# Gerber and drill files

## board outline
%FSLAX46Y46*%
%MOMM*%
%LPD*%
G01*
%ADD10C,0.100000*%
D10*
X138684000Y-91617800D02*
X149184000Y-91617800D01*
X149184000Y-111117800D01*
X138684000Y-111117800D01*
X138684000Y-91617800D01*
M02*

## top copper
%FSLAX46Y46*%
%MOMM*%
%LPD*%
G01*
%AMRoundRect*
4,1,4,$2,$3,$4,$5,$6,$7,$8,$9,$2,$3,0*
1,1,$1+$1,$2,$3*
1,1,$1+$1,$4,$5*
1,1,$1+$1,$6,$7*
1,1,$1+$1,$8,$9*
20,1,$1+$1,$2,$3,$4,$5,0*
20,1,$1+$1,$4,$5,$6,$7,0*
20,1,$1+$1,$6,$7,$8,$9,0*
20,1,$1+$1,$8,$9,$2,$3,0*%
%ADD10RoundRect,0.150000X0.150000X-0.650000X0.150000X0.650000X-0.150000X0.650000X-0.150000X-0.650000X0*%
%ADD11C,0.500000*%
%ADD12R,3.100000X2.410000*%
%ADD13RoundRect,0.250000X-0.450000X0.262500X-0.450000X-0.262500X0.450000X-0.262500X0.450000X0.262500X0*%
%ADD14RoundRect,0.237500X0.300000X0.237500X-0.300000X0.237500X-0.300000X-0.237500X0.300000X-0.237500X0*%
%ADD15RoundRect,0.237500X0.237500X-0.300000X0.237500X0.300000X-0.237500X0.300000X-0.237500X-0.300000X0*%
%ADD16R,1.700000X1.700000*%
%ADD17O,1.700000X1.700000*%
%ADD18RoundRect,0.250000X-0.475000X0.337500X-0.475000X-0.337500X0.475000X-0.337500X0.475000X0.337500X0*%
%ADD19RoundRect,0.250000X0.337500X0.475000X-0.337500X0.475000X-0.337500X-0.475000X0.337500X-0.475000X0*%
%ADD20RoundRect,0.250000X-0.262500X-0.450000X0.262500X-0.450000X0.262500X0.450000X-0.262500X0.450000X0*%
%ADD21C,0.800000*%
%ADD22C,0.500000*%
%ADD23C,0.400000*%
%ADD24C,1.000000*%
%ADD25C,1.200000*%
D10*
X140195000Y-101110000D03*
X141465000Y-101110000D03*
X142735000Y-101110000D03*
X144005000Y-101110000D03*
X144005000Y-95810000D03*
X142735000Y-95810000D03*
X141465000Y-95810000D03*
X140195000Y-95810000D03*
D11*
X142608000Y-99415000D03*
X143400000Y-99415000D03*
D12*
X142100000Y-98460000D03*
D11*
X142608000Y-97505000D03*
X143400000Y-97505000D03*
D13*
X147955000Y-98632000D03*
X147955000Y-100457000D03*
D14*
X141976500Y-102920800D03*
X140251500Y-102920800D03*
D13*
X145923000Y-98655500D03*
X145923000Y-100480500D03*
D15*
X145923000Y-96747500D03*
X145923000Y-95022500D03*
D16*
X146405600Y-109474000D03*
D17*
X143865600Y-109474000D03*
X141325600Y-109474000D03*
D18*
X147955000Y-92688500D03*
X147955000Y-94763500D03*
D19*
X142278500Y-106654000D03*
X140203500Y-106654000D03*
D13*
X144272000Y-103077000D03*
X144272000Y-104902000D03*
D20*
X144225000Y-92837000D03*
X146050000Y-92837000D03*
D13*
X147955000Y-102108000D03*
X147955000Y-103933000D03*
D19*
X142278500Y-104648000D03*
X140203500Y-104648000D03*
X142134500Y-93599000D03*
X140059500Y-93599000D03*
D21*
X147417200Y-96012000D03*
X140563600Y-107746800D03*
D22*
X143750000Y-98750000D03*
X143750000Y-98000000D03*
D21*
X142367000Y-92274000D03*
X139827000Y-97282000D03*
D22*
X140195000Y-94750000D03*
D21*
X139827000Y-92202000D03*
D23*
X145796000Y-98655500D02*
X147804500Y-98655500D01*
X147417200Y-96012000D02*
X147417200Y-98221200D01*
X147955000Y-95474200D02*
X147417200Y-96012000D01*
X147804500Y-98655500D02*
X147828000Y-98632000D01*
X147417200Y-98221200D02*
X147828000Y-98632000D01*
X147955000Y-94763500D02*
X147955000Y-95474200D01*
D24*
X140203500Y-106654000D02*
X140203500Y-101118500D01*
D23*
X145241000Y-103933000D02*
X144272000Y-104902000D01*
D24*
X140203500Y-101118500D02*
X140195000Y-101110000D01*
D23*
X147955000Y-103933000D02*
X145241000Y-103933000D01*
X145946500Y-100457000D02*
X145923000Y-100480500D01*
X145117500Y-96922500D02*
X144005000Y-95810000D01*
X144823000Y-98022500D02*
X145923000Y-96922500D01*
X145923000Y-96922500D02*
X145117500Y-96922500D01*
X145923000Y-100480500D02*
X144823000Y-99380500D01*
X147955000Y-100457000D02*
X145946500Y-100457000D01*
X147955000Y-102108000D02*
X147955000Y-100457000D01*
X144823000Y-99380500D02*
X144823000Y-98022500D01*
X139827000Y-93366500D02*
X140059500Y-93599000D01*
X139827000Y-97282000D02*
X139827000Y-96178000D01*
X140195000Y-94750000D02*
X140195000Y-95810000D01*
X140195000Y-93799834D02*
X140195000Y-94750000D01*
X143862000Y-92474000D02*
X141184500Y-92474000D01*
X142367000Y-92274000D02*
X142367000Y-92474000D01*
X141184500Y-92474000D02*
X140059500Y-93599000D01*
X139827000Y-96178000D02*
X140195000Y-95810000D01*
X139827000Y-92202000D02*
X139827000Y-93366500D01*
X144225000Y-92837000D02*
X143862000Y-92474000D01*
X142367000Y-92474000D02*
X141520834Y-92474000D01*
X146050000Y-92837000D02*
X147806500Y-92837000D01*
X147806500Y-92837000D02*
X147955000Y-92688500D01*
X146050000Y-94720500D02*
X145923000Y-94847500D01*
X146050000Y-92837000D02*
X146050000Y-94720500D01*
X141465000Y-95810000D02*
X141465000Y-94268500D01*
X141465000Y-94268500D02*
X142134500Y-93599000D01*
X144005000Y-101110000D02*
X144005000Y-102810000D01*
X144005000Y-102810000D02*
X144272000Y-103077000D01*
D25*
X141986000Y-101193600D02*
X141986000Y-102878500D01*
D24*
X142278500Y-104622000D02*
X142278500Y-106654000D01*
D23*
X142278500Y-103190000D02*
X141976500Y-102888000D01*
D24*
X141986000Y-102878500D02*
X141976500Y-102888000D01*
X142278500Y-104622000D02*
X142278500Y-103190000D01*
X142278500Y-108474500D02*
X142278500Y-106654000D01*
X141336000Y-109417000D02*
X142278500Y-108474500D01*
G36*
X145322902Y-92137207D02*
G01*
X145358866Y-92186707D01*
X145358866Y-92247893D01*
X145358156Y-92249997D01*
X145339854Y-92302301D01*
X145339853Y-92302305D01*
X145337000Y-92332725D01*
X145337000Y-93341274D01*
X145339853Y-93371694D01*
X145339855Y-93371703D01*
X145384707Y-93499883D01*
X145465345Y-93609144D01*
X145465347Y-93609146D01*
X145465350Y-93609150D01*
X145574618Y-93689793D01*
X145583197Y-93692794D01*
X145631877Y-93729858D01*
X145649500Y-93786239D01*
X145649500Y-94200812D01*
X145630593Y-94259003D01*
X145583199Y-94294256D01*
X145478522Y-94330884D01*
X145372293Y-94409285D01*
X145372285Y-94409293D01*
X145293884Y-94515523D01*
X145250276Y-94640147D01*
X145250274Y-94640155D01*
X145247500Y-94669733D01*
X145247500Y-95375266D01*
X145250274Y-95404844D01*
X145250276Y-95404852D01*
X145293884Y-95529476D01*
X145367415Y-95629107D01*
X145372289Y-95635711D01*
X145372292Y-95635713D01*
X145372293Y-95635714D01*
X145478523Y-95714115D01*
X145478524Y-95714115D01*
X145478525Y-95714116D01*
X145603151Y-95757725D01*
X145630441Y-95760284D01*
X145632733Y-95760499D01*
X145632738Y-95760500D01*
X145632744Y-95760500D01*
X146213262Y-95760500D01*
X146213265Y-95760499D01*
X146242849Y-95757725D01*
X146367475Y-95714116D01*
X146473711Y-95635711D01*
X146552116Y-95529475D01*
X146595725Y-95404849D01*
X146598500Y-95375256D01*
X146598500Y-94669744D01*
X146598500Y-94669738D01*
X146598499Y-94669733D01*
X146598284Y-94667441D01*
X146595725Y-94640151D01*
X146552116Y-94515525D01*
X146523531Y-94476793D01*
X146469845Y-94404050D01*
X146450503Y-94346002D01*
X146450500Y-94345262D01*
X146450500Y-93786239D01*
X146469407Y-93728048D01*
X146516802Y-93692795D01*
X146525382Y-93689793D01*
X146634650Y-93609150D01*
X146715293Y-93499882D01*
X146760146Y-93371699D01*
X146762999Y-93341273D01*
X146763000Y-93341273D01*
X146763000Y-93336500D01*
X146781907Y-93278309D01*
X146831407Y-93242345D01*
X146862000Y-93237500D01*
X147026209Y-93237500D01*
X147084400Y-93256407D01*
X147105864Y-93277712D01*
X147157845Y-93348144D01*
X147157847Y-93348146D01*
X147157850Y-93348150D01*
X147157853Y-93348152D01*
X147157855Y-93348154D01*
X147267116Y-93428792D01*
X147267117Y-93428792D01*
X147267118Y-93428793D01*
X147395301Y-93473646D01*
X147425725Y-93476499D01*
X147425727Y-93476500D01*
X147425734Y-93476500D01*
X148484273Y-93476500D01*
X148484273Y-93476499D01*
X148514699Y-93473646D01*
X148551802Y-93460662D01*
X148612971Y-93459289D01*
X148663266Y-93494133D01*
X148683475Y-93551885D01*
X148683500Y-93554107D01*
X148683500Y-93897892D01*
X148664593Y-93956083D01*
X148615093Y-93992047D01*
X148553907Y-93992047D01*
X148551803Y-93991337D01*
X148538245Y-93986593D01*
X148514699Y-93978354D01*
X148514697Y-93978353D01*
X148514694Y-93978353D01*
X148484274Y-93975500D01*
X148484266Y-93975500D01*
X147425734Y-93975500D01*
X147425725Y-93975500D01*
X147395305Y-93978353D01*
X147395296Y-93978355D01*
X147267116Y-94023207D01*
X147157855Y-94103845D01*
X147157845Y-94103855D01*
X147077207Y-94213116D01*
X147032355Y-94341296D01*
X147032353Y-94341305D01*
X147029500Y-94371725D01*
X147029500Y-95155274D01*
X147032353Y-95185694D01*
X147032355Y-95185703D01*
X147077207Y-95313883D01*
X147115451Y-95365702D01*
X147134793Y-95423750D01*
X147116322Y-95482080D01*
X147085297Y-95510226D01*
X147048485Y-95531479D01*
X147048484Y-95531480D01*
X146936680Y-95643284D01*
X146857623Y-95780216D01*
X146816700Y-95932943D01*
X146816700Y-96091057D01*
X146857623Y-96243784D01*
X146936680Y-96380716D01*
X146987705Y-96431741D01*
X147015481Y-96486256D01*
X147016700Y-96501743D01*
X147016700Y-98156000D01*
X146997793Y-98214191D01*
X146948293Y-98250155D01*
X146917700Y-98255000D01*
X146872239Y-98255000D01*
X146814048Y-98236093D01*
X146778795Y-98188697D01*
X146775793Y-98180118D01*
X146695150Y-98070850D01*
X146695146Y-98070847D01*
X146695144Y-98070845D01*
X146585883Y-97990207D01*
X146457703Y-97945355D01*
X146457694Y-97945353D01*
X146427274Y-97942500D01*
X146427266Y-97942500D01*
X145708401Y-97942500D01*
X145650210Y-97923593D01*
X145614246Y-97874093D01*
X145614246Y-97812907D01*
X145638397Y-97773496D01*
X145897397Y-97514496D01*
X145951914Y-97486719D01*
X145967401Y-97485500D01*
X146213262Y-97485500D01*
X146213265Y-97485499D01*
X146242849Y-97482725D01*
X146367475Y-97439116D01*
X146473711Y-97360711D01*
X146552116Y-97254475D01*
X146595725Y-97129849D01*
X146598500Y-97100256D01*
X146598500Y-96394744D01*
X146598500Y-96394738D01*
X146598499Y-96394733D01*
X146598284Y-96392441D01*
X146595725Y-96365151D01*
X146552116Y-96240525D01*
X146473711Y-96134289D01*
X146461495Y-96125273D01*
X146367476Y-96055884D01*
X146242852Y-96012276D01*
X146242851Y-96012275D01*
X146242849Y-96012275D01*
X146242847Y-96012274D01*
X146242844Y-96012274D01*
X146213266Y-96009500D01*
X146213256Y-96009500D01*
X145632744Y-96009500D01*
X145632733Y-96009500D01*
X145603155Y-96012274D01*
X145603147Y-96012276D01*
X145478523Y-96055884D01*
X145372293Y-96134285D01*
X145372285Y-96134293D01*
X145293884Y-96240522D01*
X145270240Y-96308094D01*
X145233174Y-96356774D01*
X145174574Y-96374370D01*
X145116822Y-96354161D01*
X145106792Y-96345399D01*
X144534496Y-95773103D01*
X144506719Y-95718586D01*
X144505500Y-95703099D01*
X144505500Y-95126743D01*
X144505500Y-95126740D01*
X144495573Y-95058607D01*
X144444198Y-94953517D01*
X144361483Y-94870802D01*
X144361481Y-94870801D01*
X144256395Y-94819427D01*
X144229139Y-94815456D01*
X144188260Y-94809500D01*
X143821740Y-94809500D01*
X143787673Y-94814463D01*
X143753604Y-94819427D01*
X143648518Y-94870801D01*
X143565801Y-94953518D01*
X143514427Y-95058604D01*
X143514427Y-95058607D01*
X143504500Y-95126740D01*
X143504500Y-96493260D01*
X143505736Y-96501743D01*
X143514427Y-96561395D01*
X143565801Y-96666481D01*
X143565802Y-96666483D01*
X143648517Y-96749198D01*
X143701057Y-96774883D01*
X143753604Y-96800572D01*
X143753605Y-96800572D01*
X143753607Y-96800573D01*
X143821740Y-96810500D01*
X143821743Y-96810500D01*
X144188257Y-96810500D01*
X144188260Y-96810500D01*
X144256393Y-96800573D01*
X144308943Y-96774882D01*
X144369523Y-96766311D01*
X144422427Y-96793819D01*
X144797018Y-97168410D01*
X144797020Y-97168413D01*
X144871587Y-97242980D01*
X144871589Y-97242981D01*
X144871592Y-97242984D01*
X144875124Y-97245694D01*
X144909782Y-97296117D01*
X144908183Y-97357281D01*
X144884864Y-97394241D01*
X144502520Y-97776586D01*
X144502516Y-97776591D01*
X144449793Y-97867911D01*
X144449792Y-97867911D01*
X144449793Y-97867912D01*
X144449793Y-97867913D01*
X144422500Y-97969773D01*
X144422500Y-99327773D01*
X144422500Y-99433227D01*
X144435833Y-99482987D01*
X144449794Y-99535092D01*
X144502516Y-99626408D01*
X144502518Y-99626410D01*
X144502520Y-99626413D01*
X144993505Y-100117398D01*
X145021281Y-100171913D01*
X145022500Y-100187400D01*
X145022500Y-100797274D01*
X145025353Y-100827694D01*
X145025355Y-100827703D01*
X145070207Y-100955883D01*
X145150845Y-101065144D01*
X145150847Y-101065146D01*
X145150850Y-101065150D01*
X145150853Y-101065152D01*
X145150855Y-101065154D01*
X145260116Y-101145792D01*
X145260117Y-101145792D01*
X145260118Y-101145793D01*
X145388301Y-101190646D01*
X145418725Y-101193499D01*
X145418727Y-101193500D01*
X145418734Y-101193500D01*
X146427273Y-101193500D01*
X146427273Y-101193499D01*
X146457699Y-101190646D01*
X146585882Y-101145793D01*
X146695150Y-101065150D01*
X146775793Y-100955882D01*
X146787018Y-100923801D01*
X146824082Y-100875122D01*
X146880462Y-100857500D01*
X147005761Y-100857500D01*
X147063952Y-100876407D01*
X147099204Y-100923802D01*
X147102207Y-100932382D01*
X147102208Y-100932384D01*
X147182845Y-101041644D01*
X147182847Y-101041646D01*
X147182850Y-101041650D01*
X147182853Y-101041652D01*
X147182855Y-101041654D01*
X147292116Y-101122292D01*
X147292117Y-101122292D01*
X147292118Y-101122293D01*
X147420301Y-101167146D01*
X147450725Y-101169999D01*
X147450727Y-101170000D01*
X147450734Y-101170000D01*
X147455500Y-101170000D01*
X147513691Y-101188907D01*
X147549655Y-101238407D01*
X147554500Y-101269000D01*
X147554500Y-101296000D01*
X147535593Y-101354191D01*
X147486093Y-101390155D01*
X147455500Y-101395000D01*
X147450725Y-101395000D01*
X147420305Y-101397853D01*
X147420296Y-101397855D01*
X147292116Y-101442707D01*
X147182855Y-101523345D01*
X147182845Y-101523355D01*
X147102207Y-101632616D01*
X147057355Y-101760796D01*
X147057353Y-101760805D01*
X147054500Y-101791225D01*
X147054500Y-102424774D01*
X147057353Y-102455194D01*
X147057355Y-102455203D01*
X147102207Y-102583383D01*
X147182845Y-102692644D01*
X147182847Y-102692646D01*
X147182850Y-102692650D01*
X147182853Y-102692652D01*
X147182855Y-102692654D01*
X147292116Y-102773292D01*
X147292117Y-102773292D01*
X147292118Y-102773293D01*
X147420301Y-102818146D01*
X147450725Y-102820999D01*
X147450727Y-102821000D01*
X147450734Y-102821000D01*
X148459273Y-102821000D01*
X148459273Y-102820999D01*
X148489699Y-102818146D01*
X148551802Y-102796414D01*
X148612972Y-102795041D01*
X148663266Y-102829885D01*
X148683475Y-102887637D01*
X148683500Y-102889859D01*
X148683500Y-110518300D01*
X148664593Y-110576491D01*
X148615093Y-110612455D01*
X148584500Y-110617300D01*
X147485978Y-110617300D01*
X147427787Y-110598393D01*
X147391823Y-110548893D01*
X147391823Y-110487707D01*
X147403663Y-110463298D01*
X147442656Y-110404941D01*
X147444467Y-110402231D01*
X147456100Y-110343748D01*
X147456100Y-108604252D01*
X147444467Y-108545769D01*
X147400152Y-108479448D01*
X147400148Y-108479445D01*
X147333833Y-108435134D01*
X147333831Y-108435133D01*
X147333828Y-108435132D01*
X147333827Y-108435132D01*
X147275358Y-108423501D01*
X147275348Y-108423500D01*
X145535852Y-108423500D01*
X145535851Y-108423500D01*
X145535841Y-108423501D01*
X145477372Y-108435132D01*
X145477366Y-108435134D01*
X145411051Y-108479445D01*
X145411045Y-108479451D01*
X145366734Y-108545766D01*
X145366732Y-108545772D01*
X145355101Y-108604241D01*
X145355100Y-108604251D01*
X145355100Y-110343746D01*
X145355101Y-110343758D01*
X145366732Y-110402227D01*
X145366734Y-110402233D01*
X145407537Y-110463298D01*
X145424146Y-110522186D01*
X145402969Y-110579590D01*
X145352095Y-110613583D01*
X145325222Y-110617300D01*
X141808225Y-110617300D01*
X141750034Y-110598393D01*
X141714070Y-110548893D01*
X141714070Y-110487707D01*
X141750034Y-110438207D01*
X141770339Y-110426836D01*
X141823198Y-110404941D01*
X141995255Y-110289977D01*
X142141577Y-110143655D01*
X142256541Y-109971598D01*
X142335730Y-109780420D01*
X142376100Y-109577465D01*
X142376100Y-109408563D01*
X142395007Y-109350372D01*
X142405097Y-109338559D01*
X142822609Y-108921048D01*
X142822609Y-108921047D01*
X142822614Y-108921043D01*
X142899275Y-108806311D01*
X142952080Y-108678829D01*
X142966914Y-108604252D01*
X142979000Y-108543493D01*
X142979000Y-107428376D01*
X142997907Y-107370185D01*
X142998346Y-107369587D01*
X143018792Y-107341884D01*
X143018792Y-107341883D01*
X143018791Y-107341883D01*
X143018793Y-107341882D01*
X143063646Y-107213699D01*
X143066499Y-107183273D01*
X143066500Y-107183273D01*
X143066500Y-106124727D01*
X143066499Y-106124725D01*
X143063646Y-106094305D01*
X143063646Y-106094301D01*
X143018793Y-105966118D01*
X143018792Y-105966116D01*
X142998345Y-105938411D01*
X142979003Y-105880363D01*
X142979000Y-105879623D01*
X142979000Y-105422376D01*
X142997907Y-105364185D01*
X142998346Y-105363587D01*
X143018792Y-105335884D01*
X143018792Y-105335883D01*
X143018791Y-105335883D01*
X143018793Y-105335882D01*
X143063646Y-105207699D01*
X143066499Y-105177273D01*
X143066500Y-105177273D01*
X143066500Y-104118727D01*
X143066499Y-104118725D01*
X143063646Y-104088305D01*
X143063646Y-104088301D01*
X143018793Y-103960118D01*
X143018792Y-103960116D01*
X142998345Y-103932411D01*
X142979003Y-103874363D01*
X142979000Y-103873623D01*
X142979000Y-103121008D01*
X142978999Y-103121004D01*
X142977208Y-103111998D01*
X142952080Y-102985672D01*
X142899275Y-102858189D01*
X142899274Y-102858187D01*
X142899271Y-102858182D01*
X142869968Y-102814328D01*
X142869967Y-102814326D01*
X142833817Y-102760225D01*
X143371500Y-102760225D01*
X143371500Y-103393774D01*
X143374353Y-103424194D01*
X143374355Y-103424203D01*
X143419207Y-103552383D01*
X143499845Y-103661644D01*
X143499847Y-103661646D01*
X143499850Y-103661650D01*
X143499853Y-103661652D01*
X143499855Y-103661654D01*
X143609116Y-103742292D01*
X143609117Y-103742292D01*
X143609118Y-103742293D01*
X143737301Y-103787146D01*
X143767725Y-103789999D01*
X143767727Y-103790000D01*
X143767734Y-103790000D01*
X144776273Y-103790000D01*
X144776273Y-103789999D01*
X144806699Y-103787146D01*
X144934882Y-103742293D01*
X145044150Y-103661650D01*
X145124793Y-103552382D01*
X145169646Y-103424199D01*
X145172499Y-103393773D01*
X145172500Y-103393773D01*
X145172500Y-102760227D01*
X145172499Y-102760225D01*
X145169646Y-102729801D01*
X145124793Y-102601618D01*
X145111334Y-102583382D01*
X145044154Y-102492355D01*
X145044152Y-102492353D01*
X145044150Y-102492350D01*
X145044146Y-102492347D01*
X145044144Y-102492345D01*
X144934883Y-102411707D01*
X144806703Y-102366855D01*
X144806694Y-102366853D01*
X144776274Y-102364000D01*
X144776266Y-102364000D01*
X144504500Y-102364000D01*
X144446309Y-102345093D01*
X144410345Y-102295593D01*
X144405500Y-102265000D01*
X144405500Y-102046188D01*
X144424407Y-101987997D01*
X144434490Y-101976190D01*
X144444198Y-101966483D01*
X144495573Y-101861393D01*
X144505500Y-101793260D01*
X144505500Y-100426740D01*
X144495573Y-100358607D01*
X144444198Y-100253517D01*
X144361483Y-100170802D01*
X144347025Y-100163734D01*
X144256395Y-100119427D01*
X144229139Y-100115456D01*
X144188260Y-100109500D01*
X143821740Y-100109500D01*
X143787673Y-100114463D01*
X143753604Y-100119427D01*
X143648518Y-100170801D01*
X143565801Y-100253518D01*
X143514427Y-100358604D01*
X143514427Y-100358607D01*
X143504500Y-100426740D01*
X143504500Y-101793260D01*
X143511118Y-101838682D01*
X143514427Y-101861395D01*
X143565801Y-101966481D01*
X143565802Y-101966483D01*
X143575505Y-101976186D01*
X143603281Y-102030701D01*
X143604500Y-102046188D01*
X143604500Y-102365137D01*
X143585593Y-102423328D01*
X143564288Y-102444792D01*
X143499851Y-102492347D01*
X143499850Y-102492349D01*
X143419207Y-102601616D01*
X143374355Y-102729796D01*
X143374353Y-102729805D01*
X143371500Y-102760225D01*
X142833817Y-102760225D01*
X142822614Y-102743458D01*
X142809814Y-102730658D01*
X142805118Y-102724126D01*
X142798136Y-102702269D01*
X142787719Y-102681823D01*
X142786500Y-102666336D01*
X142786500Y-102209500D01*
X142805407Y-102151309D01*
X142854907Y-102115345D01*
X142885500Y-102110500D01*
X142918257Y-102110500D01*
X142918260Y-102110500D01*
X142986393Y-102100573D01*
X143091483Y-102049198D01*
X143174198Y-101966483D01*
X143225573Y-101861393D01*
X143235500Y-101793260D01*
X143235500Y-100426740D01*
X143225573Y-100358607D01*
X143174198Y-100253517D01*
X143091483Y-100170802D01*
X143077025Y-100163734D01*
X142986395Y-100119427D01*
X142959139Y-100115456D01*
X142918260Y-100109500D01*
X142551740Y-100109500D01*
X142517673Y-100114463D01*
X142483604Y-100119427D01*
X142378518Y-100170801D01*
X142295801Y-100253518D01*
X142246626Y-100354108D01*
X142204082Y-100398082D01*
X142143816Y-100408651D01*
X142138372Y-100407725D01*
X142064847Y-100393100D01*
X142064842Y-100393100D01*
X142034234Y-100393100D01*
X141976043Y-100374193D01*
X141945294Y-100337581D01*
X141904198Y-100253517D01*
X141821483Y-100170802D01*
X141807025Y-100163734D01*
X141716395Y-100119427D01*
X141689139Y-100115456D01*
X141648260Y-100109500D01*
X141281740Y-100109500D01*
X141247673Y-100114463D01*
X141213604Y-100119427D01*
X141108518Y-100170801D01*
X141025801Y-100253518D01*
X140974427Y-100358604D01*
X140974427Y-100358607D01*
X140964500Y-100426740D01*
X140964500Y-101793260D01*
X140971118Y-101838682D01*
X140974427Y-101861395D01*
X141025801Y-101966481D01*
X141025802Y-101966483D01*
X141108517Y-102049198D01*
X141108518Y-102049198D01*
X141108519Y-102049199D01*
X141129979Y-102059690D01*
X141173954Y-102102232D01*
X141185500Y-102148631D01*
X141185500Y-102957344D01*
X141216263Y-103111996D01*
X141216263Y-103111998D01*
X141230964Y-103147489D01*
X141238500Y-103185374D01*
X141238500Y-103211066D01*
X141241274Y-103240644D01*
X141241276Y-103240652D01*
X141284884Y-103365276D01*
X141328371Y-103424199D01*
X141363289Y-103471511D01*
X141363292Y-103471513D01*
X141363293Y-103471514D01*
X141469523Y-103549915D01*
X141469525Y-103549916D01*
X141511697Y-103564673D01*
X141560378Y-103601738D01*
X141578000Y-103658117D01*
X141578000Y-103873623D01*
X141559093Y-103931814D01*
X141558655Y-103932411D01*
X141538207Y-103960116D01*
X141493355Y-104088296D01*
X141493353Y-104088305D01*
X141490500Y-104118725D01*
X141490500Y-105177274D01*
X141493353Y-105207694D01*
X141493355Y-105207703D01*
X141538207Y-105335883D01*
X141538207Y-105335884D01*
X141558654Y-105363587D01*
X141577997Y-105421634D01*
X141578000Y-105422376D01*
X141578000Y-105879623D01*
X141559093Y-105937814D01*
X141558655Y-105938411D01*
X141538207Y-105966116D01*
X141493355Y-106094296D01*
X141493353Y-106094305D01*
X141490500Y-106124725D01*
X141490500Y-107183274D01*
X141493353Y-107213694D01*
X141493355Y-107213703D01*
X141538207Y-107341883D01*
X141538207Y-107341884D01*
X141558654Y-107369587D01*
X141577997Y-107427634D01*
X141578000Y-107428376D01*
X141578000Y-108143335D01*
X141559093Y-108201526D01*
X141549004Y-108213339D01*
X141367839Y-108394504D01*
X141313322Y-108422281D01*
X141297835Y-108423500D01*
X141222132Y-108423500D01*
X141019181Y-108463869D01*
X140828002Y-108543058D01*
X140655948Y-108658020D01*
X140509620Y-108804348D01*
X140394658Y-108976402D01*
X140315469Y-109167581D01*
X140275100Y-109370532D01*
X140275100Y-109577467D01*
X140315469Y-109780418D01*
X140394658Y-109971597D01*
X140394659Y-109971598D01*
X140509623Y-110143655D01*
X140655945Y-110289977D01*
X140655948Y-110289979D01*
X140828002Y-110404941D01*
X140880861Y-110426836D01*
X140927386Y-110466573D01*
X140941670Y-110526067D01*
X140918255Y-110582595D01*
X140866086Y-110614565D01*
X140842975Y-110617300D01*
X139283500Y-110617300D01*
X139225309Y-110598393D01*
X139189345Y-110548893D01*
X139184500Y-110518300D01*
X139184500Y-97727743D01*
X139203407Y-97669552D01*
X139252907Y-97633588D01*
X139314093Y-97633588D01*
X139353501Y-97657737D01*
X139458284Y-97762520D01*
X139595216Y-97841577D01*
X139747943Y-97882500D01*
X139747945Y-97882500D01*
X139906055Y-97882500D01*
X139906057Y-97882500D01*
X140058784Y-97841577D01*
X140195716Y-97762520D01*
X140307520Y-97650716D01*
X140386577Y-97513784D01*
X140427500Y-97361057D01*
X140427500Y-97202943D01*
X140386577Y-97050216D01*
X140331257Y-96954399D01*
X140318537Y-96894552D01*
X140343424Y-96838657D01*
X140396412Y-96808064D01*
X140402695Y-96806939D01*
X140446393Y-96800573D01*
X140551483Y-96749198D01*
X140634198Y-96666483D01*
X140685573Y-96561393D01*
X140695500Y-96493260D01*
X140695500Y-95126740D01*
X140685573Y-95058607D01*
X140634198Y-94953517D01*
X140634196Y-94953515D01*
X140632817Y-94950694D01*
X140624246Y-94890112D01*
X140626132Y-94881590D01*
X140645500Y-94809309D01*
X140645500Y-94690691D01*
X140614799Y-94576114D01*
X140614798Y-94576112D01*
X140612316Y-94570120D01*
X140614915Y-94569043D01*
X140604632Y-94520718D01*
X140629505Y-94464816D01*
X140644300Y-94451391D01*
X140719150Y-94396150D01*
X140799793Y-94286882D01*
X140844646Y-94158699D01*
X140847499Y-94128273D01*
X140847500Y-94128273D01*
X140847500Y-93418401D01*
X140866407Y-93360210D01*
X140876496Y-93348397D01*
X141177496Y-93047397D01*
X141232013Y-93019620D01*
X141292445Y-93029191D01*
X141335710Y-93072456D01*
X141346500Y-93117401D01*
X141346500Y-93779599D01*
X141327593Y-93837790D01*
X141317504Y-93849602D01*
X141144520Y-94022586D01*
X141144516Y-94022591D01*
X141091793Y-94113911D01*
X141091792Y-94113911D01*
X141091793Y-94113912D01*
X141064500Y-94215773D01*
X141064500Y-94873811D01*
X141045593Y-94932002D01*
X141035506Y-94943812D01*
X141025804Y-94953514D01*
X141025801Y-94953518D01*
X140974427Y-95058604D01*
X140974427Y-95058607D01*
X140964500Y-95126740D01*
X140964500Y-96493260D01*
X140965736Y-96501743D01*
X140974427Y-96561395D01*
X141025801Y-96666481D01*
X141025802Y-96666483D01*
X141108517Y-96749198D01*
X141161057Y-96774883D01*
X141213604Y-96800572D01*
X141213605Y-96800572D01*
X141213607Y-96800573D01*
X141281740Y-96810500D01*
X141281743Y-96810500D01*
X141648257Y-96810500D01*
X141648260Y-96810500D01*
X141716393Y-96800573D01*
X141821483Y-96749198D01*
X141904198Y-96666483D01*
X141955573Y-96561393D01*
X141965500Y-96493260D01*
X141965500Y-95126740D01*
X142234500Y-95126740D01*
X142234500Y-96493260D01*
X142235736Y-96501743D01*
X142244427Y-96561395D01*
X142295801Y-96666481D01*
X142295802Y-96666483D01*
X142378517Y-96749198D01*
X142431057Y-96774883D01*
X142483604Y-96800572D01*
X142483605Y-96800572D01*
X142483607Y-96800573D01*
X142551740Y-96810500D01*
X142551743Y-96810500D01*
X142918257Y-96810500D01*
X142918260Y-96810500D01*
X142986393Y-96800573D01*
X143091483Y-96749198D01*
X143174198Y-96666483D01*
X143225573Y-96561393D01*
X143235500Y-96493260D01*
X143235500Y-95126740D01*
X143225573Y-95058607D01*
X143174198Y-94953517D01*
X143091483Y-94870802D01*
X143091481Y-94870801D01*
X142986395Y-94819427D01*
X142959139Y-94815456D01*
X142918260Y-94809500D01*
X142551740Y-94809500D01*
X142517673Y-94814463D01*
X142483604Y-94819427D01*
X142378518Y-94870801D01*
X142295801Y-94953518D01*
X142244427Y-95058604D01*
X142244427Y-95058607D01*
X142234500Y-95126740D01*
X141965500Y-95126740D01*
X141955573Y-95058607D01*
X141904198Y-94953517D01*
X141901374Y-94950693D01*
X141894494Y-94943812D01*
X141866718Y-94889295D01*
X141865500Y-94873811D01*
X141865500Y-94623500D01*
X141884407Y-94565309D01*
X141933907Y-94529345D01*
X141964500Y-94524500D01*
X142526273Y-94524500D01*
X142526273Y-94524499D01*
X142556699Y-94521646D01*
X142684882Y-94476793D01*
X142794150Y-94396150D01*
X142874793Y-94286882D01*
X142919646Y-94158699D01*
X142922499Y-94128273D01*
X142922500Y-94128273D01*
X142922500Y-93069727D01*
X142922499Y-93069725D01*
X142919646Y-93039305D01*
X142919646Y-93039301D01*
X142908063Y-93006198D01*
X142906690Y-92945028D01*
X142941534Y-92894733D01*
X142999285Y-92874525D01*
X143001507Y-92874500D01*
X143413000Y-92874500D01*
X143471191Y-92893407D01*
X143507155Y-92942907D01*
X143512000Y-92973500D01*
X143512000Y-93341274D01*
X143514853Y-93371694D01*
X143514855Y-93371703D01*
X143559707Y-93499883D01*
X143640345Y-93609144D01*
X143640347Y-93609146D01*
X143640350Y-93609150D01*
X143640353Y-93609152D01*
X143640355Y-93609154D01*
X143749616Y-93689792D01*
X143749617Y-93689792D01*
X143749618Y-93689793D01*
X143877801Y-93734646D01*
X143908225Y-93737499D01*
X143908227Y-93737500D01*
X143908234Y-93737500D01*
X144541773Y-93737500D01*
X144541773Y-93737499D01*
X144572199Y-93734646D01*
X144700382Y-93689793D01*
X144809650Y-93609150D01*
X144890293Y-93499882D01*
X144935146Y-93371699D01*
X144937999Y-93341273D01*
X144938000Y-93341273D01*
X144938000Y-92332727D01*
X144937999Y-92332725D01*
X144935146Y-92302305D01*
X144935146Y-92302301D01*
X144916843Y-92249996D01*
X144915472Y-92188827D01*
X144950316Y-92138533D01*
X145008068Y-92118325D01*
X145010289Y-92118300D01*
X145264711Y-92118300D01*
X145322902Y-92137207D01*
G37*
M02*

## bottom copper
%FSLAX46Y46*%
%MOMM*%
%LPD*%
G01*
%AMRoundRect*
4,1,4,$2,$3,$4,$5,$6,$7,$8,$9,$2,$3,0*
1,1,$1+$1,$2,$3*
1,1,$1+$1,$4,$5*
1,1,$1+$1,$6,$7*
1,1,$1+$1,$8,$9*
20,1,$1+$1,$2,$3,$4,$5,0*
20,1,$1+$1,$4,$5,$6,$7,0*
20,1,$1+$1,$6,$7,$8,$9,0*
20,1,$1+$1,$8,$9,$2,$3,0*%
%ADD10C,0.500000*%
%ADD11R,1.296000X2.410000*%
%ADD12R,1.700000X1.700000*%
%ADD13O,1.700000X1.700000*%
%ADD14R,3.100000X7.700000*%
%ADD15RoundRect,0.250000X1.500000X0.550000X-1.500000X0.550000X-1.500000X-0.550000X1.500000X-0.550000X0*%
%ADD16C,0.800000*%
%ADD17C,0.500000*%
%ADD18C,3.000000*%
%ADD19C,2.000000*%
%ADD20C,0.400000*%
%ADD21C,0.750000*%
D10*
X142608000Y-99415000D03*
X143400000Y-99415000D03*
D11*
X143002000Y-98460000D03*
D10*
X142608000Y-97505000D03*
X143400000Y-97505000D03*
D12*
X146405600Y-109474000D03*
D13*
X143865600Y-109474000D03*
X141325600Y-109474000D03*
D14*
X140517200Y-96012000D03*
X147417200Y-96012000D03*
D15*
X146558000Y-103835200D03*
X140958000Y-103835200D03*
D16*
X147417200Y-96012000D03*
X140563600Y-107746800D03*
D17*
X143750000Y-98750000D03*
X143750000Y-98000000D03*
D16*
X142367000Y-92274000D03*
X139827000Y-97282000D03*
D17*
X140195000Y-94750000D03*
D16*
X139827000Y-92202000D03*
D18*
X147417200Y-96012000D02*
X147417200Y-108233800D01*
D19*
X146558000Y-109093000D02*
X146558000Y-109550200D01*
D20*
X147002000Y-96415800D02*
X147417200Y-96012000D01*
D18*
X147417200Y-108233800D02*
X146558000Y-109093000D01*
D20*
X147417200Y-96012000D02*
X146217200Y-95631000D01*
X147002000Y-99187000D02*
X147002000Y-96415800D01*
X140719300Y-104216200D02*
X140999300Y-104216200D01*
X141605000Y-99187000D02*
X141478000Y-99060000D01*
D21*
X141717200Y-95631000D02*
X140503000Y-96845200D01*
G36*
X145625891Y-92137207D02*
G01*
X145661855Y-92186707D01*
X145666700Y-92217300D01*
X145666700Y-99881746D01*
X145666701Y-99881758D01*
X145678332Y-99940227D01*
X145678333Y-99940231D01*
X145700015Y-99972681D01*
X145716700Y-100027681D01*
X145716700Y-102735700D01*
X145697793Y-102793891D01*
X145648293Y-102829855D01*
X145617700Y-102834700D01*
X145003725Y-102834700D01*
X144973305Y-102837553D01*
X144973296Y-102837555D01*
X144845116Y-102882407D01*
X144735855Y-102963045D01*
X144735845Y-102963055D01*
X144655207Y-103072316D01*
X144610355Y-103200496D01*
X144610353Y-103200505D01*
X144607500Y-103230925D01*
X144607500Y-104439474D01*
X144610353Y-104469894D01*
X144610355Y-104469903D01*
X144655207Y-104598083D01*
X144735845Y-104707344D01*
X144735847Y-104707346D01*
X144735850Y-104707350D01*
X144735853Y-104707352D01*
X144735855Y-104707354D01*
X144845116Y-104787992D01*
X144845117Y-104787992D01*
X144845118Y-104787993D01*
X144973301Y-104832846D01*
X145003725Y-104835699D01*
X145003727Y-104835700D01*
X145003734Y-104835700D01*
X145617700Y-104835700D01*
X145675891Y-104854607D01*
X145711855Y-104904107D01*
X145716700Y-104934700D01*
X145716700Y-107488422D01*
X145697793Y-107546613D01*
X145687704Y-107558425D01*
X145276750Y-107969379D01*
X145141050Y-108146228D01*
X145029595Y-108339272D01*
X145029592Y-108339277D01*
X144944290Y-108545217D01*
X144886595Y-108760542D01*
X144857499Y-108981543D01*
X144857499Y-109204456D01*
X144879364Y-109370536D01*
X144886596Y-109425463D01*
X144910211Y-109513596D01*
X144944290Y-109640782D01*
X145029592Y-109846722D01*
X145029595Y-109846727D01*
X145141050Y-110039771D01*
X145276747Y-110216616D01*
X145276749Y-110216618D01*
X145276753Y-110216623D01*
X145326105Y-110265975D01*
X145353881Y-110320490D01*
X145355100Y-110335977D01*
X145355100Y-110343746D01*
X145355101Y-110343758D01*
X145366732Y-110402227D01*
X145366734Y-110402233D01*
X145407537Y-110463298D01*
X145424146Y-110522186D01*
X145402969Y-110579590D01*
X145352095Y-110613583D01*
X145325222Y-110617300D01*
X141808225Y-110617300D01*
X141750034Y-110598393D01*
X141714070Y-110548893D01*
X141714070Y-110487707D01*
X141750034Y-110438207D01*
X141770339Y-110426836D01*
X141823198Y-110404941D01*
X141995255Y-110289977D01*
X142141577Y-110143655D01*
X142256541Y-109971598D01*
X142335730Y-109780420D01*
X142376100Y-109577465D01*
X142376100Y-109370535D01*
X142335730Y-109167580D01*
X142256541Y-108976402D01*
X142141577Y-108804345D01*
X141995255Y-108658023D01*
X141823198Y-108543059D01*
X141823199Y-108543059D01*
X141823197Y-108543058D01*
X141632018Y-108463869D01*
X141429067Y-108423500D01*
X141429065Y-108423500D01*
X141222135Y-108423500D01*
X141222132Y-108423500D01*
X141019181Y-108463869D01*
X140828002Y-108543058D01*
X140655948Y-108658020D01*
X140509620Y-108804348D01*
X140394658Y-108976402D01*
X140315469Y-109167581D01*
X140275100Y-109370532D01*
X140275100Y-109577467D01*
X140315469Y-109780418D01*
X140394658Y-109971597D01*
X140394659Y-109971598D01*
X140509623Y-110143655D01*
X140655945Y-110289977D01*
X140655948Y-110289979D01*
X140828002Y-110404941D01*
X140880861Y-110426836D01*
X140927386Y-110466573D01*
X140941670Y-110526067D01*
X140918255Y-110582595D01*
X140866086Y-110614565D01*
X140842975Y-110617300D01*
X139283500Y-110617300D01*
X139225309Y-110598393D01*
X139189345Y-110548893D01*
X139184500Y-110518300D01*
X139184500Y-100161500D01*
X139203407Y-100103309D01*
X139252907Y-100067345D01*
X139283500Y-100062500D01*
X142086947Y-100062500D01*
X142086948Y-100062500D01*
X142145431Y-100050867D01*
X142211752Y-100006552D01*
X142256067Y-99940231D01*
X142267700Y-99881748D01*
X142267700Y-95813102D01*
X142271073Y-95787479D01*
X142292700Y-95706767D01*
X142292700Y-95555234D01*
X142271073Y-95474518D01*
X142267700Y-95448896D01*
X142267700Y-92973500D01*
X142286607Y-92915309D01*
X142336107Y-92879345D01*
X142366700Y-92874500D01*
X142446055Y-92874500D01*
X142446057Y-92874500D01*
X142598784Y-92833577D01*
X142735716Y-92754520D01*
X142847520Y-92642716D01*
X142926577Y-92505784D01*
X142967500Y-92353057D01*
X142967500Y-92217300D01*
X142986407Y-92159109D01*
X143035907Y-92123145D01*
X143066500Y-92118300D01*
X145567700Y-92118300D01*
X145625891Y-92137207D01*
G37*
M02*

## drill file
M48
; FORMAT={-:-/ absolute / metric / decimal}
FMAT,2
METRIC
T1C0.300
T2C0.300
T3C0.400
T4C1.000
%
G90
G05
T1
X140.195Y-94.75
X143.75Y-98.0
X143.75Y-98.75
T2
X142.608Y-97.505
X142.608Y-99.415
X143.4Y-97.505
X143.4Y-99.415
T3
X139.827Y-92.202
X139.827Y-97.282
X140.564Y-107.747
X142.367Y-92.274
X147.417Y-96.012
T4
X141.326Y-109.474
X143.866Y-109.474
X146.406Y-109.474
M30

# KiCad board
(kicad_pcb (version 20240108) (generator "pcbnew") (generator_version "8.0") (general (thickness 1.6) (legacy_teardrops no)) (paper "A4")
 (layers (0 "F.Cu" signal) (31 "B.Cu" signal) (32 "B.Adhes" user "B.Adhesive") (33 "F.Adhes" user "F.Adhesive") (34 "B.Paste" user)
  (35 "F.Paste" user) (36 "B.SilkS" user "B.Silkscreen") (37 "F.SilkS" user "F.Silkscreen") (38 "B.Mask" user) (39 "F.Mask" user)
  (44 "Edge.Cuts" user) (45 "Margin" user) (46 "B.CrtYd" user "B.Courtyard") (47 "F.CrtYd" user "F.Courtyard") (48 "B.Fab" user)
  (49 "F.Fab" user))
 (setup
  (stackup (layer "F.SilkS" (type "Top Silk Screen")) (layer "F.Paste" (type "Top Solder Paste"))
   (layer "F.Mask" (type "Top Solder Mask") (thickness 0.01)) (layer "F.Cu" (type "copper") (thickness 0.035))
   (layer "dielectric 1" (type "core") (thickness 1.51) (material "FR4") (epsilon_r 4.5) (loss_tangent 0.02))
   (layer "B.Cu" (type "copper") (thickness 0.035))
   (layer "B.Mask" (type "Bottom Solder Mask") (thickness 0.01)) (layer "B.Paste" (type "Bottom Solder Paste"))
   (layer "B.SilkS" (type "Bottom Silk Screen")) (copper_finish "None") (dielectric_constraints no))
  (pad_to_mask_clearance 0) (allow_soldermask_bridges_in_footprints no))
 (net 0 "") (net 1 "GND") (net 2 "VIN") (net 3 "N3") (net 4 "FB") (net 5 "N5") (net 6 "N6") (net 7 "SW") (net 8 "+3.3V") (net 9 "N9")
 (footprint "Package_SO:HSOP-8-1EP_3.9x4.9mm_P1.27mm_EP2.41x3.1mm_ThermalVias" (layer "F.Cu") (at 142.1 98.46 90)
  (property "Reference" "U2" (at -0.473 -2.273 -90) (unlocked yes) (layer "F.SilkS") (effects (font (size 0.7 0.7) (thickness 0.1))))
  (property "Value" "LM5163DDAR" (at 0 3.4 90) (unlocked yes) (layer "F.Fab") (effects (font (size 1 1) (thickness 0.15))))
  (pad "" smd roundrect (at -0.6 -0.775 90) (size 0.97 1.25) (layers "F.Paste") (roundrect_rratio 0.25))
  (pad "" smd roundrect (at -0.6 0.775 90) (size 0.97 1.25) (layers "F.Paste") (roundrect_rratio 0.25))
  (pad "" smd roundrect (at 0.6 -0.775 90) (size 0.97 1.25) (layers "F.Paste") (roundrect_rratio 0.25))
  (pad "" smd roundrect (at 0.6 0.775 90) (size 0.97 1.25) (layers "F.Paste") (roundrect_rratio 0.25))
  (pad "1" smd roundrect (at -2.65 -1.905 90) (size 1.6 0.6) (layers "F.Cu" "F.Paste" "F.Mask") (roundrect_rratio 0.25) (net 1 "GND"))
  (pad "2" smd roundrect (at -2.65 -0.635 90) (size 1.6 0.6) (layers "F.Cu" "F.Paste" "F.Mask") (roundrect_rratio 0.25) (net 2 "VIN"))
  (pad "3" smd roundrect (at -2.65 0.635 90) (size 1.6 0.6) (layers "F.Cu" "F.Paste" "F.Mask") (roundrect_rratio 0.25) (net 2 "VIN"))
  (pad "4" smd roundrect (at -2.65 1.905 90) (size 1.6 0.6) (layers "F.Cu" "F.Paste" "F.Mask") (roundrect_rratio 0.25) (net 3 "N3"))
  (pad "5" smd roundrect (at 2.65 1.905 90) (size 1.6 0.6) (layers "F.Cu" "F.Paste" "F.Mask") (roundrect_rratio 0.25) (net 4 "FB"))
  (pad "6" smd roundrect (at 2.65 0.635 90) (size 1.6 0.6) (layers "F.Cu" "F.Paste" "F.Mask") (roundrect_rratio 0.25) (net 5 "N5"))
  (pad "7" smd roundrect (at 2.65 -0.635 90) (size 1.6 0.6) (layers "F.Cu" "F.Paste" "F.Mask") (roundrect_rratio 0.25) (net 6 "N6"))
  (pad "8" smd roundrect (at 2.65 -1.905 90) (size 1.6 0.6) (layers "F.Cu" "F.Paste" "F.Mask") (roundrect_rratio 0.25) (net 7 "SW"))
  (pad "9" thru_hole circle (at -0.955 0.508 90) (size 0.5 0.5) (drill 0.3) (layers "*.Cu") (remove_unused_layers no) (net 1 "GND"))
  (pad "9" thru_hole circle (at -0.955 1.3 90) (size 0.5 0.5) (drill 0.3) (layers "*.Cu") (remove_unused_layers no) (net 1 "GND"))
  (pad "9" smd rect (at 0 0 90) (size 2.41 3.1) (layers "F.Cu" "F.Mask") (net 1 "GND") (zone_connect 2))
  (pad "9" smd rect (at 0 0.902 90) (size 2.41 1.296) (layers "B.Cu") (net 1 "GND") (zone_connect 2))
  (pad "9" thru_hole circle (at 0.955 0.508 90) (size 0.5 0.5) (drill 0.3) (layers "*.Cu") (remove_unused_layers no) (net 1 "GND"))
  (pad "9" thru_hole circle (at 0.955 1.3 90) (size 0.5 0.5) (drill 0.3) (layers "*.Cu") (remove_unused_layers no) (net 1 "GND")))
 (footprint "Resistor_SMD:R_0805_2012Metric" (layer "F.Cu") (at 147.955 99.5445 -90)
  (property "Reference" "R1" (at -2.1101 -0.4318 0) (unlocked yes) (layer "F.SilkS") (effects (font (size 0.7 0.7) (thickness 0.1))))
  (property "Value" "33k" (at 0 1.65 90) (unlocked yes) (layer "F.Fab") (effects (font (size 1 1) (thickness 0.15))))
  (pad "1" smd roundrect (at -0.9125 0 270) (size 1.025 1.4) (layers "F.Cu" "F.Paste" "F.Mask") (roundrect_rratio 0.243902439)
   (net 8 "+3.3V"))
  (pad "2" smd roundrect (at 0.9125 0 270) (size 1.025 1.4) (layers "F.Cu" "F.Paste" "F.Mask") (roundrect_rratio 0.243902439) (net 4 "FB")))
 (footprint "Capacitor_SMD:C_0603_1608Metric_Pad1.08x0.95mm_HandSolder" (layer "F.Cu") (at 141.114 102.9208 180)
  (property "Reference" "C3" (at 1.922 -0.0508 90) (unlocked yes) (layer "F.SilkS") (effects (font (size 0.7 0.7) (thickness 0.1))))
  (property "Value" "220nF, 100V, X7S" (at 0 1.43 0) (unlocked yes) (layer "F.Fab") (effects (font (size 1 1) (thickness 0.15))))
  (pad "1" smd roundrect (at -0.8625 0 180) (size 1.075 0.95) (layers "F.Cu" "F.Paste" "F.Mask") (roundrect_rratio 0.25) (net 2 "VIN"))
  (pad "2" smd roundrect (at 0.8625 0 180) (size 1.075 0.95) (layers "F.Cu" "F.Paste" "F.Mask") (roundrect_rratio 0.25) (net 1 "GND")))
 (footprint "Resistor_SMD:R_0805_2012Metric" (layer "F.Cu") (at 145.923 99.568 -90)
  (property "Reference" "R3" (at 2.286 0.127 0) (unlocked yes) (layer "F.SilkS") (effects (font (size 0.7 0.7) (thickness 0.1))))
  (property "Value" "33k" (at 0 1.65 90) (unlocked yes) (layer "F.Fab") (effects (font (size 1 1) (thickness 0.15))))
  (pad "1" smd roundrect (at -0.9125 0 270) (size 1.025 1.4) (layers "F.Cu" "F.Paste" "F.Mask") (roundrect_rratio 0.243902439)
   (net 8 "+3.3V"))
  (pad "2" smd roundrect (at 0.9125 0 270) (size 1.025 1.4) (layers "F.Cu" "F.Paste" "F.Mask") (roundrect_rratio 0.243902439) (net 4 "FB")))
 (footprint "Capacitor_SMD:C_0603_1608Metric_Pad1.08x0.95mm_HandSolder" (layer "F.Cu") (at 145.923 95.885 90)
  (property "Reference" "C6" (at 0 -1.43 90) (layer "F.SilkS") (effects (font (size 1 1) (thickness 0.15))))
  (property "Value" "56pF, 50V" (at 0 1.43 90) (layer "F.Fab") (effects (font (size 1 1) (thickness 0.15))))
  (pad "1" smd roundrect (at -0.8625 0 90) (size 1.075 0.95) (layers "F.Cu" "F.Paste" "F.Mask") (roundrect_rratio 0.25) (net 4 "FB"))
  (pad "2" smd roundrect (at 0.8625 0 90) (size 1.075 0.95) (layers "F.Cu" "F.Paste" "F.Mask") (roundrect_rratio 0.25) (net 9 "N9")))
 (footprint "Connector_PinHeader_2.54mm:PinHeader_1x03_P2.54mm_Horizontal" (layer "F.Cu") (at 146.4056 109.474 -90)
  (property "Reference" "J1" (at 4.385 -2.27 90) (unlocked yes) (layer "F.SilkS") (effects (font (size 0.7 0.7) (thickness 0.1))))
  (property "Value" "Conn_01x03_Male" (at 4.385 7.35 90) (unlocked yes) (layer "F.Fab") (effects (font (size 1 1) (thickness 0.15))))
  (pad "1" thru_hole rect (at 0 0 270) (size 1.7 1.7) (drill 1) (layers "*.Cu" "*.Mask") (remove_unused_layers no) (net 8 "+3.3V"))
  (pad "2" thru_hole oval (at 0 2.54 270) (size 1.7 1.7) (drill 1) (layers "*.Cu" "*.Mask") (remove_unused_layers no) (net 1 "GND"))
  (pad "3" thru_hole oval (at 0 5.08 270) (size 1.7 1.7) (drill 1) (layers "*.Cu" "*.Mask") (remove_unused_layers no) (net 2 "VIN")))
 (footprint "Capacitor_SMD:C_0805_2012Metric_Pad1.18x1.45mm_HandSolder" (layer "F.Cu") (at 147.955 93.726 -90)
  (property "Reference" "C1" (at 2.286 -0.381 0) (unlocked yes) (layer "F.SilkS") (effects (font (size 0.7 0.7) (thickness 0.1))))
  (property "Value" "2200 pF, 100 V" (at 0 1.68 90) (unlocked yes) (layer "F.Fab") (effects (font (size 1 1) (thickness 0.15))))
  (pad "1" smd roundrect (at -1.0375 0 270) (size 1.175 1.45) (layers "F.Cu" "F.Paste" "F.Mask") (roundrect_rratio 0.212766) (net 9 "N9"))
  (pad "2" smd roundrect (at 1.0375 0 270) (size 1.175 1.45) (layers "F.Cu" "F.Paste" "F.Mask") (roundrect_rratio 0.212766) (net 8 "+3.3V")))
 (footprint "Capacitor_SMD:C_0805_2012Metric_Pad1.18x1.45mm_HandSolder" (layer "F.Cu") (at 141.241 106.654 180)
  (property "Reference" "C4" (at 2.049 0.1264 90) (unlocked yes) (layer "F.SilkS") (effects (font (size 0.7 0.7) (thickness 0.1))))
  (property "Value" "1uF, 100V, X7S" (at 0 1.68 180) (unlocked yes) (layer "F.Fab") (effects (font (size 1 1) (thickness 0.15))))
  (pad "1" smd roundrect (at -1.0375 0 180) (size 1.175 1.45) (layers "F.Cu" "F.Paste" "F.Mask") (roundrect_rratio 0.212766) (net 2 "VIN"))
  (pad "2" smd roundrect (at 1.0375 0 180) (size 1.175 1.45) (layers "F.Cu" "F.Paste" "F.Mask") (roundrect_rratio 0.212766) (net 1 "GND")))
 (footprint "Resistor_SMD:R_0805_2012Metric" (layer "F.Cu") (at 144.272 103.9895 -90)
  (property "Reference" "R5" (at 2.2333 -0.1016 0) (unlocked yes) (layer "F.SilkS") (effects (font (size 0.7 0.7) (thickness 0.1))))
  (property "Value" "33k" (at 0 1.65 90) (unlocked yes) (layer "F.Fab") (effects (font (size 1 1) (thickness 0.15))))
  (pad "1" smd roundrect (at -0.9125 0 270) (size 1.025 1.4) (layers "F.Cu" "F.Paste" "F.Mask") (roundrect_rratio 0.243902) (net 3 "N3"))
  (pad "2" smd roundrect (at 0.9125 0 270) (size 1.025 1.4) (layers "F.Cu" "F.Paste" "F.Mask") (roundrect_rratio 0.243902) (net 1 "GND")))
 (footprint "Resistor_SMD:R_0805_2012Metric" (layer "F.Cu") (at 145.1375 92.837)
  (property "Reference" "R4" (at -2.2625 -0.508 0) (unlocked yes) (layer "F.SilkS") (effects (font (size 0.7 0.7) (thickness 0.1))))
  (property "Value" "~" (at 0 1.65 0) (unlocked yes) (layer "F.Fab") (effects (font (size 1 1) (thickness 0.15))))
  (pad "1" smd roundrect (at -0.9125 0) (size 1.025 1.4) (layers "F.Cu" "F.Paste" "F.Mask") (roundrect_rratio 0.243902) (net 7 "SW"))
  (pad "2" smd roundrect (at 0.9125 0) (size 1.025 1.4) (layers "F.Cu" "F.Paste" "F.Mask") (roundrect_rratio 0.243902) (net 9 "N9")))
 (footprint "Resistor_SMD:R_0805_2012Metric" (layer "F.Cu") (at 147.955 103.0205 -90)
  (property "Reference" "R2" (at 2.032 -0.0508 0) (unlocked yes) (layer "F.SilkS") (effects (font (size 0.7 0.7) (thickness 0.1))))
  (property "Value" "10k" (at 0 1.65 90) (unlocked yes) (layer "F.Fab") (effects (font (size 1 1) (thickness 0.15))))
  (pad "1" smd roundrect (at -0.9125 0 270) (size 1.025 1.4) (layers "F.Cu" "F.Paste" "F.Mask") (roundrect_rratio 0.243902439) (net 4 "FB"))
  (pad "2" smd roundrect (at 0.9125 0 270) (size 1.025 1.4) (layers "F.Cu" "F.Paste" "F.Mask") (roundrect_rratio 0.243902439) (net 1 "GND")))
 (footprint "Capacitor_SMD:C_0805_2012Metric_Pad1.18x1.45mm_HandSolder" (layer "F.Cu") (at 141.241 104.648 180)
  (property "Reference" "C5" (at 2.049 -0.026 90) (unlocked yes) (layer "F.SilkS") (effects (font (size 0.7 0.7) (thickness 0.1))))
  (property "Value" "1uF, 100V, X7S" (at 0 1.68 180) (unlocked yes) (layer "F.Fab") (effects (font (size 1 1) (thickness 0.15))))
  (pad "1" smd roundrect (at -1.0375 0 180) (size 1.175 1.45) (layers "F.Cu" "F.Paste" "F.Mask") (roundrect_rratio 0.212766) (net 2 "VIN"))
  (pad "2" smd roundrect (at 1.0375 0 180) (size 1.175 1.45) (layers "F.Cu" "F.Paste" "F.Mask") (roundrect_rratio 0.212766) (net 1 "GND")))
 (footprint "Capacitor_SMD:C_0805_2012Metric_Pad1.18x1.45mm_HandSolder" (layer "F.Cu") (at 141.097 93.599 180)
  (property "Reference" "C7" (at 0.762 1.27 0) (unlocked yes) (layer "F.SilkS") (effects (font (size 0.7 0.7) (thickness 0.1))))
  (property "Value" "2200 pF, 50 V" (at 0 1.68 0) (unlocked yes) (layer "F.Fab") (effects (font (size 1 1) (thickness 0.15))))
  (pad "1" smd roundrect (at -1.0375 0 180) (size 1.175 1.45) (layers "F.Cu" "F.Paste" "F.Mask") (roundrect_rratio 0.212766) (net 6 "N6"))
  (pad "2" smd roundrect (at 1.0375 0 180) (size 1.175 1.45) (layers "F.Cu" "F.Paste" "F.Mask") (roundrect_rratio 0.212766) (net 7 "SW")))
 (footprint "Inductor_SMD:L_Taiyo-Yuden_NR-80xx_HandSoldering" (layer "B.Cu") (at 143.9672 96.012)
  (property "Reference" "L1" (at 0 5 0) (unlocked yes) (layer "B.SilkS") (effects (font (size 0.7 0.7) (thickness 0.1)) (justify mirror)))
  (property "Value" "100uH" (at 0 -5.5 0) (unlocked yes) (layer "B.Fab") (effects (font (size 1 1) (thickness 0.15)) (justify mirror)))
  (pad "1" smd rect (at -3.45 0) (size 3.1 7.7) (layers "B.Cu" "B.Paste" "B.Mask") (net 7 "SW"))
  (pad "2" smd rect (at 3.45 0) (size 3.1 7.7) (layers "B.Cu" "B.Paste" "B.Mask") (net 8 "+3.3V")))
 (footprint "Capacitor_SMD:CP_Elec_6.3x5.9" (layer "B.Cu") (at 143.758 103.8352 180)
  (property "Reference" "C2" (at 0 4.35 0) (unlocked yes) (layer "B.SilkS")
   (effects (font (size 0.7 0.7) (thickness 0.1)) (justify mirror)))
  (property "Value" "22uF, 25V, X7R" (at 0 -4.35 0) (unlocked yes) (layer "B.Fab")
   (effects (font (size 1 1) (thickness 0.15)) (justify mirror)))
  (pad "1" smd roundrect (at -2.8 0 180) (size 3.5 1.6) (layers "B.Cu" "B.Paste" "B.Mask") (roundrect_rratio 0.15625) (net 8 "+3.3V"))
  (pad "2" smd roundrect (at 2.8 0 180) (size 3.5 1.6) (layers "B.Cu" "B.Paste" "B.Mask") (roundrect_rratio 0.15625) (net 1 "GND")))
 (gr_rect (start 138.684 91.6178) (end 149.184 111.1178) (stroke (width 0.1) (type solid)) (fill none) (layer "Edge.Cuts"))
 (segment (start 145.796 98.6555) (end 147.8045 98.6555) (width 0.4) (layer "F.Cu") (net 8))
 (segment (start 147.4172 96.012) (end 147.4172 98.2212) (width 0.4) (layer "F.Cu") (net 8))
 (segment (start 147.955 95.4742) (end 147.4172 96.012) (width 0.4) (layer "F.Cu") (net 8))
 (segment (start 147.8045 98.6555) (end 147.828 98.632) (width 0.4) (layer "F.Cu") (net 8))
 (segment (start 147.4172 98.2212) (end 147.828 98.632) (width 0.4) (layer "F.Cu") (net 8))
 (segment (start 147.955 94.7635) (end 147.955 95.4742) (width 0.4) (layer "F.Cu") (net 8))
 (via (at 147.4172 96.012) (size 0.8) (drill 0.4) (layers "F.Cu" "B.Cu") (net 8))
 (segment (start 147.4172 96.012) (end 147.4172 108.2338) (width 3) (layer "B.Cu") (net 8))
 (segment (start 146.558 109.093) (end 146.558 109.5502) (width 2) (layer "B.Cu") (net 8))
 (segment (start 147.002 96.4158) (end 147.4172 96.012) (width 0.4) (layer "B.Cu") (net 8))
 (segment (start 147.4172 108.2338) (end 146.558 109.093) (width 3) (layer "B.Cu") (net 8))
 (segment (start 147.4172 96.012) (end 146.2172 95.631) (width 0.4) (layer "B.Cu") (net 8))
 (segment (start 147.002 99.187) (end 147.002 96.4158) (width 0.4) (layer "B.Cu") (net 8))
 (segment (start 140.2035 106.654) (end 140.2035 101.1185) (width 1) (layer "F.Cu") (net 1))
 (segment (start 145.241 103.933) (end 144.272 104.902) (width 0.4) (layer "F.Cu") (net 1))
 (segment (start 140.2035 101.1185) (end 140.195 101.11) (width 1) (layer "F.Cu") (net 1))
 (segment (start 147.955 103.933) (end 145.241 103.933) (width 0.4) (layer "F.Cu") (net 1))
 (via (at 140.5636 107.7468) (size 0.8) (drill 0.4) (layers "F.Cu" "B.Cu") (free yes) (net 1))
 (via (at 143.75 98.75) (size 0.5) (drill 0.3) (layers "F.Cu" "B.Cu") (free yes) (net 1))
 (via (at 143.75 98) (size 0.5) (drill 0.3) (layers "F.Cu" "B.Cu") (free yes) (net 1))
 (segment (start 140.7193 104.2162) (end 140.9993 104.2162) (width 0.4) (layer "B.Cu") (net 1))
 (segment (start 145.9465 100.457) (end 145.923 100.4805) (width 0.4) (layer "F.Cu") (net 4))
 (segment (start 145.1175 96.9225) (end 144.005 95.81) (width 0.4) (layer "F.Cu") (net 4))
 (segment (start 144.823 98.0225) (end 145.923 96.9225) (width 0.4) (layer "F.Cu") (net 4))
 (segment (start 145.923 96.9225) (end 145.1175 96.9225) (width 0.4) (layer "F.Cu") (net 4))
 (segment (start 145.923 100.4805) (end 144.823 99.3805) (width 0.4) (layer "F.Cu") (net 4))
 (segment (start 147.955 100.457) (end 145.9465 100.457) (width 0.4) (layer "F.Cu") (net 4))
 (segment (start 147.955 102.108) (end 147.955 100.457) (width 0.4) (layer "F.Cu") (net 4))
 (segment (start 144.823 99.3805) (end 144.823 98.0225) (width 0.4) (layer "F.Cu") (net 4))
 (segment (start 139.827 93.3665) (end 140.0595 93.599) (width 0.4) (layer "F.Cu") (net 7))
 (segment (start 139.827 97.282) (end 139.827 96.178) (width 0.4) (layer "F.Cu") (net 7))
 (segment (start 140.195 94.75) (end 140.195 95.81) (width 0.4) (layer "F.Cu") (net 7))
 (segment (start 140.195 93.799834) (end 140.195 94.75) (width 0.4) (layer "F.Cu") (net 7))
 (segment (start 143.862 92.474) (end 141.1845 92.474) (width 0.4) (layer "F.Cu") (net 7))
 (segment (start 142.367 92.274) (end 142.367 92.474) (width 0.4) (layer "F.Cu") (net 7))
 (segment (start 141.1845 92.474) (end 140.0595 93.599) (width 0.4) (layer "F.Cu") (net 7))
 (segment (start 139.827 96.178) (end 140.195 95.81) (width 0.4) (layer "F.Cu") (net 7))
 (segment (start 139.827 92.202) (end 139.827 93.3665) (width 0.4) (layer "F.Cu") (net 7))
 (segment (start 144.225 92.837) (end 143.862 92.474) (width 0.4) (layer "F.Cu") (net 7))
 (segment (start 142.367 92.474) (end 141.520834 92.474) (width 0.4) (layer "F.Cu") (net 7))
 (via (at 142.367 92.274) (size 0.8) (drill 0.4) (layers "F.Cu" "B.Cu") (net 7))
 (via (at 139.827 97.282) (size 0.8) (drill 0.4) (layers "F.Cu" "B.Cu") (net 7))
 (via (at 140.195 94.75) (size 0.5) (drill 0.3) (layers "F.Cu" "B.Cu") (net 7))
 (via (at 139.827 92.202) (size 0.8) (drill 0.4) (layers "F.Cu" "B.Cu") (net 7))
 (segment (start 141.605 99.187) (end 141.478 99.06) (width 0.4) (layer "B.Cu") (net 7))
 (segment (start 141.7172 95.631) (end 140.503 96.8452) (width 0.75) (layer "B.Cu") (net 7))
 (segment (start 146.05 92.837) (end 147.8065 92.837) (width 0.4) (layer "F.Cu") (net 9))
 (segment (start 147.8065 92.837) (end 147.955 92.6885) (width 0.4) (layer "F.Cu") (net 9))
 (segment (start 146.05 94.7205) (end 145.923 94.8475) (width 0.4) (layer "F.Cu") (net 9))
 (segment (start 146.05 92.837) (end 146.05 94.7205) (width 0.4) (layer "F.Cu") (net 9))
 (segment (start 141.465 95.81) (end 141.465 94.2685) (width 0.4) (layer "F.Cu") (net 6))
 (segment (start 141.465 94.2685) (end 142.1345 93.599) (width 0.4) (layer "F.Cu") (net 6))
 (segment (start 144.005 101.11) (end 144.005 102.81) (width 0.4) (layer "F.Cu") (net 3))
 (segment (start 144.005 102.81) (end 144.272 103.077) (width 0.4) (layer "F.Cu") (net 3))
 (segment (start 141.986 101.1936) (end 141.986 102.8785) (width 1.2) (layer "F.Cu") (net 2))
 (segment (start 142.2785 104.622) (end 142.2785 106.654) (width 1) (layer "F.Cu") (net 2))
 (segment (start 142.2785 103.19) (end 141.9765 102.888) (width 0.4) (layer "F.Cu") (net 2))
 (segment (start 141.986 102.8785) (end 141.9765 102.888) (width 1) (layer "F.Cu") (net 2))
 (segment (start 142.2785 104.622) (end 142.2785 103.19) (width 1) (layer "F.Cu") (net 2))
 (segment (start 142.2785 108.4745) (end 142.2785 106.654) (width 1) (layer "F.Cu") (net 2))
 (segment (start 141.336 109.417) (end 142.2785 108.4745) (width 1) (layer "F.Cu") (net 2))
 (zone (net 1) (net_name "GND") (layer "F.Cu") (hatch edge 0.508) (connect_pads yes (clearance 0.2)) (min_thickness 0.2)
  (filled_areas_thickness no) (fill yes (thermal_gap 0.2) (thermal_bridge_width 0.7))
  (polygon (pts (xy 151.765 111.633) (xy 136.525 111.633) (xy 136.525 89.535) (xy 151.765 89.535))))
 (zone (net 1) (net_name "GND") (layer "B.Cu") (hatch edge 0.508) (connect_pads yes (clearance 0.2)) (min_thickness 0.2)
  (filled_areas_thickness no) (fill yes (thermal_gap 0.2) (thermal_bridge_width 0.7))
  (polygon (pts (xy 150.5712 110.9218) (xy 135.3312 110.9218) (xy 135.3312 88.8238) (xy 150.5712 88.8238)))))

